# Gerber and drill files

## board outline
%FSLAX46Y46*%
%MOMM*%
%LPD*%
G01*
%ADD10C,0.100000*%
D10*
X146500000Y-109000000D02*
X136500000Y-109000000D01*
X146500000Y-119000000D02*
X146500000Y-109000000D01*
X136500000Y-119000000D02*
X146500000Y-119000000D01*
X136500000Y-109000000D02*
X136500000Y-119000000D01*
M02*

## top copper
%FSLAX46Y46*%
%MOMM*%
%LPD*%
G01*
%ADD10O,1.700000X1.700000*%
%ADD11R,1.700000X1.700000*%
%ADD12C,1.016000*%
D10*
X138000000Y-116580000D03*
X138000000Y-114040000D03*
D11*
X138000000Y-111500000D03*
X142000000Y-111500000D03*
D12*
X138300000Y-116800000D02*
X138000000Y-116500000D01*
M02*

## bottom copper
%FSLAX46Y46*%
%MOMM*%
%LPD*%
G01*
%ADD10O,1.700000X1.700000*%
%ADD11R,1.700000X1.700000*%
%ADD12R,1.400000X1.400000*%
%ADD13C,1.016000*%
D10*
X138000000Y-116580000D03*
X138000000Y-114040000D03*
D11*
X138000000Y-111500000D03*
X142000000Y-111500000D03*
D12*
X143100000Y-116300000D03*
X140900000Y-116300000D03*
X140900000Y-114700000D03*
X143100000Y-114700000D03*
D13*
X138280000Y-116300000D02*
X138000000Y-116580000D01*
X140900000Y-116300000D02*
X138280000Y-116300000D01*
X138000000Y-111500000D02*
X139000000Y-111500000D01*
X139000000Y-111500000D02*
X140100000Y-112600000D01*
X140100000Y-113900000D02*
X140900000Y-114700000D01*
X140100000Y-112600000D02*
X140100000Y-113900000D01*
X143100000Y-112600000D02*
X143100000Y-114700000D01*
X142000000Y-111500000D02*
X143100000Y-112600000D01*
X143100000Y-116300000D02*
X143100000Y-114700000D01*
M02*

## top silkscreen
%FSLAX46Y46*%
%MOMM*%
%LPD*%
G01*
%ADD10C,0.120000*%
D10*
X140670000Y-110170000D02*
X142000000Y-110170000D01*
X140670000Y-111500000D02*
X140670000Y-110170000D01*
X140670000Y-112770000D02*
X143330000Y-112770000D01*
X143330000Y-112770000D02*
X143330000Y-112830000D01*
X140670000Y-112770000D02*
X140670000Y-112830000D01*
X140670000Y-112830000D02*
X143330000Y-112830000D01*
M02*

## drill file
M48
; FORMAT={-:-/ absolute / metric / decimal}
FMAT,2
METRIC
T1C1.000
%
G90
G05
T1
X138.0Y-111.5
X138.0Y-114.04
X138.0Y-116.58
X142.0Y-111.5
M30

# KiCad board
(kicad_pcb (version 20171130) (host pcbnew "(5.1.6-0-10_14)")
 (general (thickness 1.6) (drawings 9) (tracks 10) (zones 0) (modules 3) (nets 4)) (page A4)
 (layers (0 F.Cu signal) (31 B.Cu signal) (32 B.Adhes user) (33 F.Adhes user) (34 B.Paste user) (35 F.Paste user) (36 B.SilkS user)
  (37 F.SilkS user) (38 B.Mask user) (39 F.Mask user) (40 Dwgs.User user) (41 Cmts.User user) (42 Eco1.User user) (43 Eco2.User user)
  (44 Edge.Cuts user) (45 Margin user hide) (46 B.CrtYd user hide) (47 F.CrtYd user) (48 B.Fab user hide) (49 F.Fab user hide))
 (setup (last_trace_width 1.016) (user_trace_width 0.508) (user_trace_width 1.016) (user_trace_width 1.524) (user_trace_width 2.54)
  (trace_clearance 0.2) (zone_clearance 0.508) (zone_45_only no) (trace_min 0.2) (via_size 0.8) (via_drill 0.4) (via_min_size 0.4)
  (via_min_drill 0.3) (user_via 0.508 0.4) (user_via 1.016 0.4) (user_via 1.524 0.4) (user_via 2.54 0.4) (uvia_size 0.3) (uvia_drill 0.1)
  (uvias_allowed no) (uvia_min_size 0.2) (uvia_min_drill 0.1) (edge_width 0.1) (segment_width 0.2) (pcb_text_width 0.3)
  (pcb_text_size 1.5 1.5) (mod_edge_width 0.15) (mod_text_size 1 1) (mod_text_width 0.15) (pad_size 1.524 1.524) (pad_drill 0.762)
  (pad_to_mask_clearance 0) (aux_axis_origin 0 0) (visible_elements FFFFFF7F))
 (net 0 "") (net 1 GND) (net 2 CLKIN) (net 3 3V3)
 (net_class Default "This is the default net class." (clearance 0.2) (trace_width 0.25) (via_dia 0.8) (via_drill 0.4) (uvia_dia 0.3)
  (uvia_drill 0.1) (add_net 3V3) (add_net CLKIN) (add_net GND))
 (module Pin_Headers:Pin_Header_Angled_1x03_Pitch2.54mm (layer B.Cu) (at 138 111.5 180)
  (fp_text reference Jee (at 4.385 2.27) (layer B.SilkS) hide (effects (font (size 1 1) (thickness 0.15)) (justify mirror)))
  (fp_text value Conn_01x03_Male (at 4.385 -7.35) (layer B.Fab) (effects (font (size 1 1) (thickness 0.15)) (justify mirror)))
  (pad 3 thru_hole oval (at 0 -5.08 180) (size 1.7 1.7) (drill 1) (layers *.Cu *.Mask) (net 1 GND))
  (pad 2 thru_hole oval (at 0 -2.54 180) (size 1.7 1.7) (drill 1) (layers *.Cu *.Mask))
  (pad 1 thru_hole rect (at 0 0 180) (size 1.7 1.7) (drill 1) (layers *.Cu *.Mask) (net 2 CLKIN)))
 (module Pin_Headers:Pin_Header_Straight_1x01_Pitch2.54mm (layer F.Cu) (at 142 111.5)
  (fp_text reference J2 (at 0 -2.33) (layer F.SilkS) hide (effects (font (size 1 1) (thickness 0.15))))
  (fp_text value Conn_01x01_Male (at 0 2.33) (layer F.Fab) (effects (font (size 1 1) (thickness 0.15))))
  (fp_line (start -1.33 -1.33) (end 0 -1.33) (layer F.SilkS) (width 0.12))
  (fp_line (start -1.33 0) (end -1.33 -1.33) (layer F.SilkS) (width 0.12))
  (fp_line (start -1.33 1.27) (end 1.33 1.27) (layer F.SilkS) (width 0.12))
  (fp_line (start 1.33 1.27) (end 1.33 1.33) (layer F.SilkS) (width 0.12))
  (fp_line (start -1.33 1.27) (end -1.33 1.33) (layer F.SilkS) (width 0.12))
  (fp_line (start -1.33 1.33) (end 1.33 1.33) (layer F.SilkS) (width 0.12))
  (pad 1 thru_hole rect (at 0 0) (size 1.7 1.7) (drill 1) (layers *.Cu *.Mask) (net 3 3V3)))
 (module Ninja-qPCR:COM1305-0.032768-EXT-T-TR (layer B.Cu) (at 142 115.5 180)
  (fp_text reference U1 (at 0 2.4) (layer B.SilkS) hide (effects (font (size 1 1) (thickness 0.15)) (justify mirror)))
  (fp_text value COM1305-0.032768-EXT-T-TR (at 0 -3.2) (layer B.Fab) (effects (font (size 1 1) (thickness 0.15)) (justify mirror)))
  (pad 1 smd rect (at -1.1 -0.8 180) (size 1.4 1.4) (layers B.Cu B.Paste B.Mask) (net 3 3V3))
  (pad 2 smd rect (at 1.1 -0.8 180) (size 1.4 1.4) (layers B.Cu B.Paste B.Mask) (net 1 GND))
  (pad 3 smd rect (at 1.1 0.8 180) (size 1.4 1.4) (layers B.Cu B.Paste B.Mask) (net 2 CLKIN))
  (pad 4 smd rect (at -1.1 0.8 180) (size 1.4 1.4) (layers B.Cu B.Paste B.Mask) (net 3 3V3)))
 (gr_line (start 146.5 109) (end 136.5 109) (layer Edge.Cuts) (width 0.1))
 (gr_line (start 146.5 119) (end 146.5 109) (layer Edge.Cuts) (width 0.1))
 (gr_line (start 136.5 119) (end 146.5 119) (layer Edge.Cuts) (width 0.1))
 (gr_line (start 136.5 109) (end 136.5 119) (layer Edge.Cuts) (width 0.1))
 (segment (start 138.3 116.8) (end 138 116.5) (width 1.016) (layer F.Cu) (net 1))
 (segment (start 138.28 116.3) (end 138 116.58) (width 1.016) (layer B.Cu) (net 1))
 (segment (start 140.9 116.3) (end 138.28 116.3) (width 1.016) (layer B.Cu) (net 1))
 (segment (start 138 111.5) (end 139 111.5) (width 1.016) (layer B.Cu) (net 2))
 (segment (start 139 111.5) (end 140.1 112.6) (width 1.016) (layer B.Cu) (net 2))
 (segment (start 140.1 113.9) (end 140.9 114.7) (width 1.016) (layer B.Cu) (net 2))
 (segment (start 140.1 112.6) (end 140.1 113.9) (width 1.016) (layer B.Cu) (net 2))
 (segment (start 143.1 112.6) (end 143.1 114.7) (width 1.016) (layer B.Cu) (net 3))
 (segment (start 142 111.5) (end 143.1 112.6) (width 1.016) (layer B.Cu) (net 3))
 (segment (start 143.1 116.3) (end 143.1 114.7) (width 1.016) (layer B.Cu) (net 3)))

